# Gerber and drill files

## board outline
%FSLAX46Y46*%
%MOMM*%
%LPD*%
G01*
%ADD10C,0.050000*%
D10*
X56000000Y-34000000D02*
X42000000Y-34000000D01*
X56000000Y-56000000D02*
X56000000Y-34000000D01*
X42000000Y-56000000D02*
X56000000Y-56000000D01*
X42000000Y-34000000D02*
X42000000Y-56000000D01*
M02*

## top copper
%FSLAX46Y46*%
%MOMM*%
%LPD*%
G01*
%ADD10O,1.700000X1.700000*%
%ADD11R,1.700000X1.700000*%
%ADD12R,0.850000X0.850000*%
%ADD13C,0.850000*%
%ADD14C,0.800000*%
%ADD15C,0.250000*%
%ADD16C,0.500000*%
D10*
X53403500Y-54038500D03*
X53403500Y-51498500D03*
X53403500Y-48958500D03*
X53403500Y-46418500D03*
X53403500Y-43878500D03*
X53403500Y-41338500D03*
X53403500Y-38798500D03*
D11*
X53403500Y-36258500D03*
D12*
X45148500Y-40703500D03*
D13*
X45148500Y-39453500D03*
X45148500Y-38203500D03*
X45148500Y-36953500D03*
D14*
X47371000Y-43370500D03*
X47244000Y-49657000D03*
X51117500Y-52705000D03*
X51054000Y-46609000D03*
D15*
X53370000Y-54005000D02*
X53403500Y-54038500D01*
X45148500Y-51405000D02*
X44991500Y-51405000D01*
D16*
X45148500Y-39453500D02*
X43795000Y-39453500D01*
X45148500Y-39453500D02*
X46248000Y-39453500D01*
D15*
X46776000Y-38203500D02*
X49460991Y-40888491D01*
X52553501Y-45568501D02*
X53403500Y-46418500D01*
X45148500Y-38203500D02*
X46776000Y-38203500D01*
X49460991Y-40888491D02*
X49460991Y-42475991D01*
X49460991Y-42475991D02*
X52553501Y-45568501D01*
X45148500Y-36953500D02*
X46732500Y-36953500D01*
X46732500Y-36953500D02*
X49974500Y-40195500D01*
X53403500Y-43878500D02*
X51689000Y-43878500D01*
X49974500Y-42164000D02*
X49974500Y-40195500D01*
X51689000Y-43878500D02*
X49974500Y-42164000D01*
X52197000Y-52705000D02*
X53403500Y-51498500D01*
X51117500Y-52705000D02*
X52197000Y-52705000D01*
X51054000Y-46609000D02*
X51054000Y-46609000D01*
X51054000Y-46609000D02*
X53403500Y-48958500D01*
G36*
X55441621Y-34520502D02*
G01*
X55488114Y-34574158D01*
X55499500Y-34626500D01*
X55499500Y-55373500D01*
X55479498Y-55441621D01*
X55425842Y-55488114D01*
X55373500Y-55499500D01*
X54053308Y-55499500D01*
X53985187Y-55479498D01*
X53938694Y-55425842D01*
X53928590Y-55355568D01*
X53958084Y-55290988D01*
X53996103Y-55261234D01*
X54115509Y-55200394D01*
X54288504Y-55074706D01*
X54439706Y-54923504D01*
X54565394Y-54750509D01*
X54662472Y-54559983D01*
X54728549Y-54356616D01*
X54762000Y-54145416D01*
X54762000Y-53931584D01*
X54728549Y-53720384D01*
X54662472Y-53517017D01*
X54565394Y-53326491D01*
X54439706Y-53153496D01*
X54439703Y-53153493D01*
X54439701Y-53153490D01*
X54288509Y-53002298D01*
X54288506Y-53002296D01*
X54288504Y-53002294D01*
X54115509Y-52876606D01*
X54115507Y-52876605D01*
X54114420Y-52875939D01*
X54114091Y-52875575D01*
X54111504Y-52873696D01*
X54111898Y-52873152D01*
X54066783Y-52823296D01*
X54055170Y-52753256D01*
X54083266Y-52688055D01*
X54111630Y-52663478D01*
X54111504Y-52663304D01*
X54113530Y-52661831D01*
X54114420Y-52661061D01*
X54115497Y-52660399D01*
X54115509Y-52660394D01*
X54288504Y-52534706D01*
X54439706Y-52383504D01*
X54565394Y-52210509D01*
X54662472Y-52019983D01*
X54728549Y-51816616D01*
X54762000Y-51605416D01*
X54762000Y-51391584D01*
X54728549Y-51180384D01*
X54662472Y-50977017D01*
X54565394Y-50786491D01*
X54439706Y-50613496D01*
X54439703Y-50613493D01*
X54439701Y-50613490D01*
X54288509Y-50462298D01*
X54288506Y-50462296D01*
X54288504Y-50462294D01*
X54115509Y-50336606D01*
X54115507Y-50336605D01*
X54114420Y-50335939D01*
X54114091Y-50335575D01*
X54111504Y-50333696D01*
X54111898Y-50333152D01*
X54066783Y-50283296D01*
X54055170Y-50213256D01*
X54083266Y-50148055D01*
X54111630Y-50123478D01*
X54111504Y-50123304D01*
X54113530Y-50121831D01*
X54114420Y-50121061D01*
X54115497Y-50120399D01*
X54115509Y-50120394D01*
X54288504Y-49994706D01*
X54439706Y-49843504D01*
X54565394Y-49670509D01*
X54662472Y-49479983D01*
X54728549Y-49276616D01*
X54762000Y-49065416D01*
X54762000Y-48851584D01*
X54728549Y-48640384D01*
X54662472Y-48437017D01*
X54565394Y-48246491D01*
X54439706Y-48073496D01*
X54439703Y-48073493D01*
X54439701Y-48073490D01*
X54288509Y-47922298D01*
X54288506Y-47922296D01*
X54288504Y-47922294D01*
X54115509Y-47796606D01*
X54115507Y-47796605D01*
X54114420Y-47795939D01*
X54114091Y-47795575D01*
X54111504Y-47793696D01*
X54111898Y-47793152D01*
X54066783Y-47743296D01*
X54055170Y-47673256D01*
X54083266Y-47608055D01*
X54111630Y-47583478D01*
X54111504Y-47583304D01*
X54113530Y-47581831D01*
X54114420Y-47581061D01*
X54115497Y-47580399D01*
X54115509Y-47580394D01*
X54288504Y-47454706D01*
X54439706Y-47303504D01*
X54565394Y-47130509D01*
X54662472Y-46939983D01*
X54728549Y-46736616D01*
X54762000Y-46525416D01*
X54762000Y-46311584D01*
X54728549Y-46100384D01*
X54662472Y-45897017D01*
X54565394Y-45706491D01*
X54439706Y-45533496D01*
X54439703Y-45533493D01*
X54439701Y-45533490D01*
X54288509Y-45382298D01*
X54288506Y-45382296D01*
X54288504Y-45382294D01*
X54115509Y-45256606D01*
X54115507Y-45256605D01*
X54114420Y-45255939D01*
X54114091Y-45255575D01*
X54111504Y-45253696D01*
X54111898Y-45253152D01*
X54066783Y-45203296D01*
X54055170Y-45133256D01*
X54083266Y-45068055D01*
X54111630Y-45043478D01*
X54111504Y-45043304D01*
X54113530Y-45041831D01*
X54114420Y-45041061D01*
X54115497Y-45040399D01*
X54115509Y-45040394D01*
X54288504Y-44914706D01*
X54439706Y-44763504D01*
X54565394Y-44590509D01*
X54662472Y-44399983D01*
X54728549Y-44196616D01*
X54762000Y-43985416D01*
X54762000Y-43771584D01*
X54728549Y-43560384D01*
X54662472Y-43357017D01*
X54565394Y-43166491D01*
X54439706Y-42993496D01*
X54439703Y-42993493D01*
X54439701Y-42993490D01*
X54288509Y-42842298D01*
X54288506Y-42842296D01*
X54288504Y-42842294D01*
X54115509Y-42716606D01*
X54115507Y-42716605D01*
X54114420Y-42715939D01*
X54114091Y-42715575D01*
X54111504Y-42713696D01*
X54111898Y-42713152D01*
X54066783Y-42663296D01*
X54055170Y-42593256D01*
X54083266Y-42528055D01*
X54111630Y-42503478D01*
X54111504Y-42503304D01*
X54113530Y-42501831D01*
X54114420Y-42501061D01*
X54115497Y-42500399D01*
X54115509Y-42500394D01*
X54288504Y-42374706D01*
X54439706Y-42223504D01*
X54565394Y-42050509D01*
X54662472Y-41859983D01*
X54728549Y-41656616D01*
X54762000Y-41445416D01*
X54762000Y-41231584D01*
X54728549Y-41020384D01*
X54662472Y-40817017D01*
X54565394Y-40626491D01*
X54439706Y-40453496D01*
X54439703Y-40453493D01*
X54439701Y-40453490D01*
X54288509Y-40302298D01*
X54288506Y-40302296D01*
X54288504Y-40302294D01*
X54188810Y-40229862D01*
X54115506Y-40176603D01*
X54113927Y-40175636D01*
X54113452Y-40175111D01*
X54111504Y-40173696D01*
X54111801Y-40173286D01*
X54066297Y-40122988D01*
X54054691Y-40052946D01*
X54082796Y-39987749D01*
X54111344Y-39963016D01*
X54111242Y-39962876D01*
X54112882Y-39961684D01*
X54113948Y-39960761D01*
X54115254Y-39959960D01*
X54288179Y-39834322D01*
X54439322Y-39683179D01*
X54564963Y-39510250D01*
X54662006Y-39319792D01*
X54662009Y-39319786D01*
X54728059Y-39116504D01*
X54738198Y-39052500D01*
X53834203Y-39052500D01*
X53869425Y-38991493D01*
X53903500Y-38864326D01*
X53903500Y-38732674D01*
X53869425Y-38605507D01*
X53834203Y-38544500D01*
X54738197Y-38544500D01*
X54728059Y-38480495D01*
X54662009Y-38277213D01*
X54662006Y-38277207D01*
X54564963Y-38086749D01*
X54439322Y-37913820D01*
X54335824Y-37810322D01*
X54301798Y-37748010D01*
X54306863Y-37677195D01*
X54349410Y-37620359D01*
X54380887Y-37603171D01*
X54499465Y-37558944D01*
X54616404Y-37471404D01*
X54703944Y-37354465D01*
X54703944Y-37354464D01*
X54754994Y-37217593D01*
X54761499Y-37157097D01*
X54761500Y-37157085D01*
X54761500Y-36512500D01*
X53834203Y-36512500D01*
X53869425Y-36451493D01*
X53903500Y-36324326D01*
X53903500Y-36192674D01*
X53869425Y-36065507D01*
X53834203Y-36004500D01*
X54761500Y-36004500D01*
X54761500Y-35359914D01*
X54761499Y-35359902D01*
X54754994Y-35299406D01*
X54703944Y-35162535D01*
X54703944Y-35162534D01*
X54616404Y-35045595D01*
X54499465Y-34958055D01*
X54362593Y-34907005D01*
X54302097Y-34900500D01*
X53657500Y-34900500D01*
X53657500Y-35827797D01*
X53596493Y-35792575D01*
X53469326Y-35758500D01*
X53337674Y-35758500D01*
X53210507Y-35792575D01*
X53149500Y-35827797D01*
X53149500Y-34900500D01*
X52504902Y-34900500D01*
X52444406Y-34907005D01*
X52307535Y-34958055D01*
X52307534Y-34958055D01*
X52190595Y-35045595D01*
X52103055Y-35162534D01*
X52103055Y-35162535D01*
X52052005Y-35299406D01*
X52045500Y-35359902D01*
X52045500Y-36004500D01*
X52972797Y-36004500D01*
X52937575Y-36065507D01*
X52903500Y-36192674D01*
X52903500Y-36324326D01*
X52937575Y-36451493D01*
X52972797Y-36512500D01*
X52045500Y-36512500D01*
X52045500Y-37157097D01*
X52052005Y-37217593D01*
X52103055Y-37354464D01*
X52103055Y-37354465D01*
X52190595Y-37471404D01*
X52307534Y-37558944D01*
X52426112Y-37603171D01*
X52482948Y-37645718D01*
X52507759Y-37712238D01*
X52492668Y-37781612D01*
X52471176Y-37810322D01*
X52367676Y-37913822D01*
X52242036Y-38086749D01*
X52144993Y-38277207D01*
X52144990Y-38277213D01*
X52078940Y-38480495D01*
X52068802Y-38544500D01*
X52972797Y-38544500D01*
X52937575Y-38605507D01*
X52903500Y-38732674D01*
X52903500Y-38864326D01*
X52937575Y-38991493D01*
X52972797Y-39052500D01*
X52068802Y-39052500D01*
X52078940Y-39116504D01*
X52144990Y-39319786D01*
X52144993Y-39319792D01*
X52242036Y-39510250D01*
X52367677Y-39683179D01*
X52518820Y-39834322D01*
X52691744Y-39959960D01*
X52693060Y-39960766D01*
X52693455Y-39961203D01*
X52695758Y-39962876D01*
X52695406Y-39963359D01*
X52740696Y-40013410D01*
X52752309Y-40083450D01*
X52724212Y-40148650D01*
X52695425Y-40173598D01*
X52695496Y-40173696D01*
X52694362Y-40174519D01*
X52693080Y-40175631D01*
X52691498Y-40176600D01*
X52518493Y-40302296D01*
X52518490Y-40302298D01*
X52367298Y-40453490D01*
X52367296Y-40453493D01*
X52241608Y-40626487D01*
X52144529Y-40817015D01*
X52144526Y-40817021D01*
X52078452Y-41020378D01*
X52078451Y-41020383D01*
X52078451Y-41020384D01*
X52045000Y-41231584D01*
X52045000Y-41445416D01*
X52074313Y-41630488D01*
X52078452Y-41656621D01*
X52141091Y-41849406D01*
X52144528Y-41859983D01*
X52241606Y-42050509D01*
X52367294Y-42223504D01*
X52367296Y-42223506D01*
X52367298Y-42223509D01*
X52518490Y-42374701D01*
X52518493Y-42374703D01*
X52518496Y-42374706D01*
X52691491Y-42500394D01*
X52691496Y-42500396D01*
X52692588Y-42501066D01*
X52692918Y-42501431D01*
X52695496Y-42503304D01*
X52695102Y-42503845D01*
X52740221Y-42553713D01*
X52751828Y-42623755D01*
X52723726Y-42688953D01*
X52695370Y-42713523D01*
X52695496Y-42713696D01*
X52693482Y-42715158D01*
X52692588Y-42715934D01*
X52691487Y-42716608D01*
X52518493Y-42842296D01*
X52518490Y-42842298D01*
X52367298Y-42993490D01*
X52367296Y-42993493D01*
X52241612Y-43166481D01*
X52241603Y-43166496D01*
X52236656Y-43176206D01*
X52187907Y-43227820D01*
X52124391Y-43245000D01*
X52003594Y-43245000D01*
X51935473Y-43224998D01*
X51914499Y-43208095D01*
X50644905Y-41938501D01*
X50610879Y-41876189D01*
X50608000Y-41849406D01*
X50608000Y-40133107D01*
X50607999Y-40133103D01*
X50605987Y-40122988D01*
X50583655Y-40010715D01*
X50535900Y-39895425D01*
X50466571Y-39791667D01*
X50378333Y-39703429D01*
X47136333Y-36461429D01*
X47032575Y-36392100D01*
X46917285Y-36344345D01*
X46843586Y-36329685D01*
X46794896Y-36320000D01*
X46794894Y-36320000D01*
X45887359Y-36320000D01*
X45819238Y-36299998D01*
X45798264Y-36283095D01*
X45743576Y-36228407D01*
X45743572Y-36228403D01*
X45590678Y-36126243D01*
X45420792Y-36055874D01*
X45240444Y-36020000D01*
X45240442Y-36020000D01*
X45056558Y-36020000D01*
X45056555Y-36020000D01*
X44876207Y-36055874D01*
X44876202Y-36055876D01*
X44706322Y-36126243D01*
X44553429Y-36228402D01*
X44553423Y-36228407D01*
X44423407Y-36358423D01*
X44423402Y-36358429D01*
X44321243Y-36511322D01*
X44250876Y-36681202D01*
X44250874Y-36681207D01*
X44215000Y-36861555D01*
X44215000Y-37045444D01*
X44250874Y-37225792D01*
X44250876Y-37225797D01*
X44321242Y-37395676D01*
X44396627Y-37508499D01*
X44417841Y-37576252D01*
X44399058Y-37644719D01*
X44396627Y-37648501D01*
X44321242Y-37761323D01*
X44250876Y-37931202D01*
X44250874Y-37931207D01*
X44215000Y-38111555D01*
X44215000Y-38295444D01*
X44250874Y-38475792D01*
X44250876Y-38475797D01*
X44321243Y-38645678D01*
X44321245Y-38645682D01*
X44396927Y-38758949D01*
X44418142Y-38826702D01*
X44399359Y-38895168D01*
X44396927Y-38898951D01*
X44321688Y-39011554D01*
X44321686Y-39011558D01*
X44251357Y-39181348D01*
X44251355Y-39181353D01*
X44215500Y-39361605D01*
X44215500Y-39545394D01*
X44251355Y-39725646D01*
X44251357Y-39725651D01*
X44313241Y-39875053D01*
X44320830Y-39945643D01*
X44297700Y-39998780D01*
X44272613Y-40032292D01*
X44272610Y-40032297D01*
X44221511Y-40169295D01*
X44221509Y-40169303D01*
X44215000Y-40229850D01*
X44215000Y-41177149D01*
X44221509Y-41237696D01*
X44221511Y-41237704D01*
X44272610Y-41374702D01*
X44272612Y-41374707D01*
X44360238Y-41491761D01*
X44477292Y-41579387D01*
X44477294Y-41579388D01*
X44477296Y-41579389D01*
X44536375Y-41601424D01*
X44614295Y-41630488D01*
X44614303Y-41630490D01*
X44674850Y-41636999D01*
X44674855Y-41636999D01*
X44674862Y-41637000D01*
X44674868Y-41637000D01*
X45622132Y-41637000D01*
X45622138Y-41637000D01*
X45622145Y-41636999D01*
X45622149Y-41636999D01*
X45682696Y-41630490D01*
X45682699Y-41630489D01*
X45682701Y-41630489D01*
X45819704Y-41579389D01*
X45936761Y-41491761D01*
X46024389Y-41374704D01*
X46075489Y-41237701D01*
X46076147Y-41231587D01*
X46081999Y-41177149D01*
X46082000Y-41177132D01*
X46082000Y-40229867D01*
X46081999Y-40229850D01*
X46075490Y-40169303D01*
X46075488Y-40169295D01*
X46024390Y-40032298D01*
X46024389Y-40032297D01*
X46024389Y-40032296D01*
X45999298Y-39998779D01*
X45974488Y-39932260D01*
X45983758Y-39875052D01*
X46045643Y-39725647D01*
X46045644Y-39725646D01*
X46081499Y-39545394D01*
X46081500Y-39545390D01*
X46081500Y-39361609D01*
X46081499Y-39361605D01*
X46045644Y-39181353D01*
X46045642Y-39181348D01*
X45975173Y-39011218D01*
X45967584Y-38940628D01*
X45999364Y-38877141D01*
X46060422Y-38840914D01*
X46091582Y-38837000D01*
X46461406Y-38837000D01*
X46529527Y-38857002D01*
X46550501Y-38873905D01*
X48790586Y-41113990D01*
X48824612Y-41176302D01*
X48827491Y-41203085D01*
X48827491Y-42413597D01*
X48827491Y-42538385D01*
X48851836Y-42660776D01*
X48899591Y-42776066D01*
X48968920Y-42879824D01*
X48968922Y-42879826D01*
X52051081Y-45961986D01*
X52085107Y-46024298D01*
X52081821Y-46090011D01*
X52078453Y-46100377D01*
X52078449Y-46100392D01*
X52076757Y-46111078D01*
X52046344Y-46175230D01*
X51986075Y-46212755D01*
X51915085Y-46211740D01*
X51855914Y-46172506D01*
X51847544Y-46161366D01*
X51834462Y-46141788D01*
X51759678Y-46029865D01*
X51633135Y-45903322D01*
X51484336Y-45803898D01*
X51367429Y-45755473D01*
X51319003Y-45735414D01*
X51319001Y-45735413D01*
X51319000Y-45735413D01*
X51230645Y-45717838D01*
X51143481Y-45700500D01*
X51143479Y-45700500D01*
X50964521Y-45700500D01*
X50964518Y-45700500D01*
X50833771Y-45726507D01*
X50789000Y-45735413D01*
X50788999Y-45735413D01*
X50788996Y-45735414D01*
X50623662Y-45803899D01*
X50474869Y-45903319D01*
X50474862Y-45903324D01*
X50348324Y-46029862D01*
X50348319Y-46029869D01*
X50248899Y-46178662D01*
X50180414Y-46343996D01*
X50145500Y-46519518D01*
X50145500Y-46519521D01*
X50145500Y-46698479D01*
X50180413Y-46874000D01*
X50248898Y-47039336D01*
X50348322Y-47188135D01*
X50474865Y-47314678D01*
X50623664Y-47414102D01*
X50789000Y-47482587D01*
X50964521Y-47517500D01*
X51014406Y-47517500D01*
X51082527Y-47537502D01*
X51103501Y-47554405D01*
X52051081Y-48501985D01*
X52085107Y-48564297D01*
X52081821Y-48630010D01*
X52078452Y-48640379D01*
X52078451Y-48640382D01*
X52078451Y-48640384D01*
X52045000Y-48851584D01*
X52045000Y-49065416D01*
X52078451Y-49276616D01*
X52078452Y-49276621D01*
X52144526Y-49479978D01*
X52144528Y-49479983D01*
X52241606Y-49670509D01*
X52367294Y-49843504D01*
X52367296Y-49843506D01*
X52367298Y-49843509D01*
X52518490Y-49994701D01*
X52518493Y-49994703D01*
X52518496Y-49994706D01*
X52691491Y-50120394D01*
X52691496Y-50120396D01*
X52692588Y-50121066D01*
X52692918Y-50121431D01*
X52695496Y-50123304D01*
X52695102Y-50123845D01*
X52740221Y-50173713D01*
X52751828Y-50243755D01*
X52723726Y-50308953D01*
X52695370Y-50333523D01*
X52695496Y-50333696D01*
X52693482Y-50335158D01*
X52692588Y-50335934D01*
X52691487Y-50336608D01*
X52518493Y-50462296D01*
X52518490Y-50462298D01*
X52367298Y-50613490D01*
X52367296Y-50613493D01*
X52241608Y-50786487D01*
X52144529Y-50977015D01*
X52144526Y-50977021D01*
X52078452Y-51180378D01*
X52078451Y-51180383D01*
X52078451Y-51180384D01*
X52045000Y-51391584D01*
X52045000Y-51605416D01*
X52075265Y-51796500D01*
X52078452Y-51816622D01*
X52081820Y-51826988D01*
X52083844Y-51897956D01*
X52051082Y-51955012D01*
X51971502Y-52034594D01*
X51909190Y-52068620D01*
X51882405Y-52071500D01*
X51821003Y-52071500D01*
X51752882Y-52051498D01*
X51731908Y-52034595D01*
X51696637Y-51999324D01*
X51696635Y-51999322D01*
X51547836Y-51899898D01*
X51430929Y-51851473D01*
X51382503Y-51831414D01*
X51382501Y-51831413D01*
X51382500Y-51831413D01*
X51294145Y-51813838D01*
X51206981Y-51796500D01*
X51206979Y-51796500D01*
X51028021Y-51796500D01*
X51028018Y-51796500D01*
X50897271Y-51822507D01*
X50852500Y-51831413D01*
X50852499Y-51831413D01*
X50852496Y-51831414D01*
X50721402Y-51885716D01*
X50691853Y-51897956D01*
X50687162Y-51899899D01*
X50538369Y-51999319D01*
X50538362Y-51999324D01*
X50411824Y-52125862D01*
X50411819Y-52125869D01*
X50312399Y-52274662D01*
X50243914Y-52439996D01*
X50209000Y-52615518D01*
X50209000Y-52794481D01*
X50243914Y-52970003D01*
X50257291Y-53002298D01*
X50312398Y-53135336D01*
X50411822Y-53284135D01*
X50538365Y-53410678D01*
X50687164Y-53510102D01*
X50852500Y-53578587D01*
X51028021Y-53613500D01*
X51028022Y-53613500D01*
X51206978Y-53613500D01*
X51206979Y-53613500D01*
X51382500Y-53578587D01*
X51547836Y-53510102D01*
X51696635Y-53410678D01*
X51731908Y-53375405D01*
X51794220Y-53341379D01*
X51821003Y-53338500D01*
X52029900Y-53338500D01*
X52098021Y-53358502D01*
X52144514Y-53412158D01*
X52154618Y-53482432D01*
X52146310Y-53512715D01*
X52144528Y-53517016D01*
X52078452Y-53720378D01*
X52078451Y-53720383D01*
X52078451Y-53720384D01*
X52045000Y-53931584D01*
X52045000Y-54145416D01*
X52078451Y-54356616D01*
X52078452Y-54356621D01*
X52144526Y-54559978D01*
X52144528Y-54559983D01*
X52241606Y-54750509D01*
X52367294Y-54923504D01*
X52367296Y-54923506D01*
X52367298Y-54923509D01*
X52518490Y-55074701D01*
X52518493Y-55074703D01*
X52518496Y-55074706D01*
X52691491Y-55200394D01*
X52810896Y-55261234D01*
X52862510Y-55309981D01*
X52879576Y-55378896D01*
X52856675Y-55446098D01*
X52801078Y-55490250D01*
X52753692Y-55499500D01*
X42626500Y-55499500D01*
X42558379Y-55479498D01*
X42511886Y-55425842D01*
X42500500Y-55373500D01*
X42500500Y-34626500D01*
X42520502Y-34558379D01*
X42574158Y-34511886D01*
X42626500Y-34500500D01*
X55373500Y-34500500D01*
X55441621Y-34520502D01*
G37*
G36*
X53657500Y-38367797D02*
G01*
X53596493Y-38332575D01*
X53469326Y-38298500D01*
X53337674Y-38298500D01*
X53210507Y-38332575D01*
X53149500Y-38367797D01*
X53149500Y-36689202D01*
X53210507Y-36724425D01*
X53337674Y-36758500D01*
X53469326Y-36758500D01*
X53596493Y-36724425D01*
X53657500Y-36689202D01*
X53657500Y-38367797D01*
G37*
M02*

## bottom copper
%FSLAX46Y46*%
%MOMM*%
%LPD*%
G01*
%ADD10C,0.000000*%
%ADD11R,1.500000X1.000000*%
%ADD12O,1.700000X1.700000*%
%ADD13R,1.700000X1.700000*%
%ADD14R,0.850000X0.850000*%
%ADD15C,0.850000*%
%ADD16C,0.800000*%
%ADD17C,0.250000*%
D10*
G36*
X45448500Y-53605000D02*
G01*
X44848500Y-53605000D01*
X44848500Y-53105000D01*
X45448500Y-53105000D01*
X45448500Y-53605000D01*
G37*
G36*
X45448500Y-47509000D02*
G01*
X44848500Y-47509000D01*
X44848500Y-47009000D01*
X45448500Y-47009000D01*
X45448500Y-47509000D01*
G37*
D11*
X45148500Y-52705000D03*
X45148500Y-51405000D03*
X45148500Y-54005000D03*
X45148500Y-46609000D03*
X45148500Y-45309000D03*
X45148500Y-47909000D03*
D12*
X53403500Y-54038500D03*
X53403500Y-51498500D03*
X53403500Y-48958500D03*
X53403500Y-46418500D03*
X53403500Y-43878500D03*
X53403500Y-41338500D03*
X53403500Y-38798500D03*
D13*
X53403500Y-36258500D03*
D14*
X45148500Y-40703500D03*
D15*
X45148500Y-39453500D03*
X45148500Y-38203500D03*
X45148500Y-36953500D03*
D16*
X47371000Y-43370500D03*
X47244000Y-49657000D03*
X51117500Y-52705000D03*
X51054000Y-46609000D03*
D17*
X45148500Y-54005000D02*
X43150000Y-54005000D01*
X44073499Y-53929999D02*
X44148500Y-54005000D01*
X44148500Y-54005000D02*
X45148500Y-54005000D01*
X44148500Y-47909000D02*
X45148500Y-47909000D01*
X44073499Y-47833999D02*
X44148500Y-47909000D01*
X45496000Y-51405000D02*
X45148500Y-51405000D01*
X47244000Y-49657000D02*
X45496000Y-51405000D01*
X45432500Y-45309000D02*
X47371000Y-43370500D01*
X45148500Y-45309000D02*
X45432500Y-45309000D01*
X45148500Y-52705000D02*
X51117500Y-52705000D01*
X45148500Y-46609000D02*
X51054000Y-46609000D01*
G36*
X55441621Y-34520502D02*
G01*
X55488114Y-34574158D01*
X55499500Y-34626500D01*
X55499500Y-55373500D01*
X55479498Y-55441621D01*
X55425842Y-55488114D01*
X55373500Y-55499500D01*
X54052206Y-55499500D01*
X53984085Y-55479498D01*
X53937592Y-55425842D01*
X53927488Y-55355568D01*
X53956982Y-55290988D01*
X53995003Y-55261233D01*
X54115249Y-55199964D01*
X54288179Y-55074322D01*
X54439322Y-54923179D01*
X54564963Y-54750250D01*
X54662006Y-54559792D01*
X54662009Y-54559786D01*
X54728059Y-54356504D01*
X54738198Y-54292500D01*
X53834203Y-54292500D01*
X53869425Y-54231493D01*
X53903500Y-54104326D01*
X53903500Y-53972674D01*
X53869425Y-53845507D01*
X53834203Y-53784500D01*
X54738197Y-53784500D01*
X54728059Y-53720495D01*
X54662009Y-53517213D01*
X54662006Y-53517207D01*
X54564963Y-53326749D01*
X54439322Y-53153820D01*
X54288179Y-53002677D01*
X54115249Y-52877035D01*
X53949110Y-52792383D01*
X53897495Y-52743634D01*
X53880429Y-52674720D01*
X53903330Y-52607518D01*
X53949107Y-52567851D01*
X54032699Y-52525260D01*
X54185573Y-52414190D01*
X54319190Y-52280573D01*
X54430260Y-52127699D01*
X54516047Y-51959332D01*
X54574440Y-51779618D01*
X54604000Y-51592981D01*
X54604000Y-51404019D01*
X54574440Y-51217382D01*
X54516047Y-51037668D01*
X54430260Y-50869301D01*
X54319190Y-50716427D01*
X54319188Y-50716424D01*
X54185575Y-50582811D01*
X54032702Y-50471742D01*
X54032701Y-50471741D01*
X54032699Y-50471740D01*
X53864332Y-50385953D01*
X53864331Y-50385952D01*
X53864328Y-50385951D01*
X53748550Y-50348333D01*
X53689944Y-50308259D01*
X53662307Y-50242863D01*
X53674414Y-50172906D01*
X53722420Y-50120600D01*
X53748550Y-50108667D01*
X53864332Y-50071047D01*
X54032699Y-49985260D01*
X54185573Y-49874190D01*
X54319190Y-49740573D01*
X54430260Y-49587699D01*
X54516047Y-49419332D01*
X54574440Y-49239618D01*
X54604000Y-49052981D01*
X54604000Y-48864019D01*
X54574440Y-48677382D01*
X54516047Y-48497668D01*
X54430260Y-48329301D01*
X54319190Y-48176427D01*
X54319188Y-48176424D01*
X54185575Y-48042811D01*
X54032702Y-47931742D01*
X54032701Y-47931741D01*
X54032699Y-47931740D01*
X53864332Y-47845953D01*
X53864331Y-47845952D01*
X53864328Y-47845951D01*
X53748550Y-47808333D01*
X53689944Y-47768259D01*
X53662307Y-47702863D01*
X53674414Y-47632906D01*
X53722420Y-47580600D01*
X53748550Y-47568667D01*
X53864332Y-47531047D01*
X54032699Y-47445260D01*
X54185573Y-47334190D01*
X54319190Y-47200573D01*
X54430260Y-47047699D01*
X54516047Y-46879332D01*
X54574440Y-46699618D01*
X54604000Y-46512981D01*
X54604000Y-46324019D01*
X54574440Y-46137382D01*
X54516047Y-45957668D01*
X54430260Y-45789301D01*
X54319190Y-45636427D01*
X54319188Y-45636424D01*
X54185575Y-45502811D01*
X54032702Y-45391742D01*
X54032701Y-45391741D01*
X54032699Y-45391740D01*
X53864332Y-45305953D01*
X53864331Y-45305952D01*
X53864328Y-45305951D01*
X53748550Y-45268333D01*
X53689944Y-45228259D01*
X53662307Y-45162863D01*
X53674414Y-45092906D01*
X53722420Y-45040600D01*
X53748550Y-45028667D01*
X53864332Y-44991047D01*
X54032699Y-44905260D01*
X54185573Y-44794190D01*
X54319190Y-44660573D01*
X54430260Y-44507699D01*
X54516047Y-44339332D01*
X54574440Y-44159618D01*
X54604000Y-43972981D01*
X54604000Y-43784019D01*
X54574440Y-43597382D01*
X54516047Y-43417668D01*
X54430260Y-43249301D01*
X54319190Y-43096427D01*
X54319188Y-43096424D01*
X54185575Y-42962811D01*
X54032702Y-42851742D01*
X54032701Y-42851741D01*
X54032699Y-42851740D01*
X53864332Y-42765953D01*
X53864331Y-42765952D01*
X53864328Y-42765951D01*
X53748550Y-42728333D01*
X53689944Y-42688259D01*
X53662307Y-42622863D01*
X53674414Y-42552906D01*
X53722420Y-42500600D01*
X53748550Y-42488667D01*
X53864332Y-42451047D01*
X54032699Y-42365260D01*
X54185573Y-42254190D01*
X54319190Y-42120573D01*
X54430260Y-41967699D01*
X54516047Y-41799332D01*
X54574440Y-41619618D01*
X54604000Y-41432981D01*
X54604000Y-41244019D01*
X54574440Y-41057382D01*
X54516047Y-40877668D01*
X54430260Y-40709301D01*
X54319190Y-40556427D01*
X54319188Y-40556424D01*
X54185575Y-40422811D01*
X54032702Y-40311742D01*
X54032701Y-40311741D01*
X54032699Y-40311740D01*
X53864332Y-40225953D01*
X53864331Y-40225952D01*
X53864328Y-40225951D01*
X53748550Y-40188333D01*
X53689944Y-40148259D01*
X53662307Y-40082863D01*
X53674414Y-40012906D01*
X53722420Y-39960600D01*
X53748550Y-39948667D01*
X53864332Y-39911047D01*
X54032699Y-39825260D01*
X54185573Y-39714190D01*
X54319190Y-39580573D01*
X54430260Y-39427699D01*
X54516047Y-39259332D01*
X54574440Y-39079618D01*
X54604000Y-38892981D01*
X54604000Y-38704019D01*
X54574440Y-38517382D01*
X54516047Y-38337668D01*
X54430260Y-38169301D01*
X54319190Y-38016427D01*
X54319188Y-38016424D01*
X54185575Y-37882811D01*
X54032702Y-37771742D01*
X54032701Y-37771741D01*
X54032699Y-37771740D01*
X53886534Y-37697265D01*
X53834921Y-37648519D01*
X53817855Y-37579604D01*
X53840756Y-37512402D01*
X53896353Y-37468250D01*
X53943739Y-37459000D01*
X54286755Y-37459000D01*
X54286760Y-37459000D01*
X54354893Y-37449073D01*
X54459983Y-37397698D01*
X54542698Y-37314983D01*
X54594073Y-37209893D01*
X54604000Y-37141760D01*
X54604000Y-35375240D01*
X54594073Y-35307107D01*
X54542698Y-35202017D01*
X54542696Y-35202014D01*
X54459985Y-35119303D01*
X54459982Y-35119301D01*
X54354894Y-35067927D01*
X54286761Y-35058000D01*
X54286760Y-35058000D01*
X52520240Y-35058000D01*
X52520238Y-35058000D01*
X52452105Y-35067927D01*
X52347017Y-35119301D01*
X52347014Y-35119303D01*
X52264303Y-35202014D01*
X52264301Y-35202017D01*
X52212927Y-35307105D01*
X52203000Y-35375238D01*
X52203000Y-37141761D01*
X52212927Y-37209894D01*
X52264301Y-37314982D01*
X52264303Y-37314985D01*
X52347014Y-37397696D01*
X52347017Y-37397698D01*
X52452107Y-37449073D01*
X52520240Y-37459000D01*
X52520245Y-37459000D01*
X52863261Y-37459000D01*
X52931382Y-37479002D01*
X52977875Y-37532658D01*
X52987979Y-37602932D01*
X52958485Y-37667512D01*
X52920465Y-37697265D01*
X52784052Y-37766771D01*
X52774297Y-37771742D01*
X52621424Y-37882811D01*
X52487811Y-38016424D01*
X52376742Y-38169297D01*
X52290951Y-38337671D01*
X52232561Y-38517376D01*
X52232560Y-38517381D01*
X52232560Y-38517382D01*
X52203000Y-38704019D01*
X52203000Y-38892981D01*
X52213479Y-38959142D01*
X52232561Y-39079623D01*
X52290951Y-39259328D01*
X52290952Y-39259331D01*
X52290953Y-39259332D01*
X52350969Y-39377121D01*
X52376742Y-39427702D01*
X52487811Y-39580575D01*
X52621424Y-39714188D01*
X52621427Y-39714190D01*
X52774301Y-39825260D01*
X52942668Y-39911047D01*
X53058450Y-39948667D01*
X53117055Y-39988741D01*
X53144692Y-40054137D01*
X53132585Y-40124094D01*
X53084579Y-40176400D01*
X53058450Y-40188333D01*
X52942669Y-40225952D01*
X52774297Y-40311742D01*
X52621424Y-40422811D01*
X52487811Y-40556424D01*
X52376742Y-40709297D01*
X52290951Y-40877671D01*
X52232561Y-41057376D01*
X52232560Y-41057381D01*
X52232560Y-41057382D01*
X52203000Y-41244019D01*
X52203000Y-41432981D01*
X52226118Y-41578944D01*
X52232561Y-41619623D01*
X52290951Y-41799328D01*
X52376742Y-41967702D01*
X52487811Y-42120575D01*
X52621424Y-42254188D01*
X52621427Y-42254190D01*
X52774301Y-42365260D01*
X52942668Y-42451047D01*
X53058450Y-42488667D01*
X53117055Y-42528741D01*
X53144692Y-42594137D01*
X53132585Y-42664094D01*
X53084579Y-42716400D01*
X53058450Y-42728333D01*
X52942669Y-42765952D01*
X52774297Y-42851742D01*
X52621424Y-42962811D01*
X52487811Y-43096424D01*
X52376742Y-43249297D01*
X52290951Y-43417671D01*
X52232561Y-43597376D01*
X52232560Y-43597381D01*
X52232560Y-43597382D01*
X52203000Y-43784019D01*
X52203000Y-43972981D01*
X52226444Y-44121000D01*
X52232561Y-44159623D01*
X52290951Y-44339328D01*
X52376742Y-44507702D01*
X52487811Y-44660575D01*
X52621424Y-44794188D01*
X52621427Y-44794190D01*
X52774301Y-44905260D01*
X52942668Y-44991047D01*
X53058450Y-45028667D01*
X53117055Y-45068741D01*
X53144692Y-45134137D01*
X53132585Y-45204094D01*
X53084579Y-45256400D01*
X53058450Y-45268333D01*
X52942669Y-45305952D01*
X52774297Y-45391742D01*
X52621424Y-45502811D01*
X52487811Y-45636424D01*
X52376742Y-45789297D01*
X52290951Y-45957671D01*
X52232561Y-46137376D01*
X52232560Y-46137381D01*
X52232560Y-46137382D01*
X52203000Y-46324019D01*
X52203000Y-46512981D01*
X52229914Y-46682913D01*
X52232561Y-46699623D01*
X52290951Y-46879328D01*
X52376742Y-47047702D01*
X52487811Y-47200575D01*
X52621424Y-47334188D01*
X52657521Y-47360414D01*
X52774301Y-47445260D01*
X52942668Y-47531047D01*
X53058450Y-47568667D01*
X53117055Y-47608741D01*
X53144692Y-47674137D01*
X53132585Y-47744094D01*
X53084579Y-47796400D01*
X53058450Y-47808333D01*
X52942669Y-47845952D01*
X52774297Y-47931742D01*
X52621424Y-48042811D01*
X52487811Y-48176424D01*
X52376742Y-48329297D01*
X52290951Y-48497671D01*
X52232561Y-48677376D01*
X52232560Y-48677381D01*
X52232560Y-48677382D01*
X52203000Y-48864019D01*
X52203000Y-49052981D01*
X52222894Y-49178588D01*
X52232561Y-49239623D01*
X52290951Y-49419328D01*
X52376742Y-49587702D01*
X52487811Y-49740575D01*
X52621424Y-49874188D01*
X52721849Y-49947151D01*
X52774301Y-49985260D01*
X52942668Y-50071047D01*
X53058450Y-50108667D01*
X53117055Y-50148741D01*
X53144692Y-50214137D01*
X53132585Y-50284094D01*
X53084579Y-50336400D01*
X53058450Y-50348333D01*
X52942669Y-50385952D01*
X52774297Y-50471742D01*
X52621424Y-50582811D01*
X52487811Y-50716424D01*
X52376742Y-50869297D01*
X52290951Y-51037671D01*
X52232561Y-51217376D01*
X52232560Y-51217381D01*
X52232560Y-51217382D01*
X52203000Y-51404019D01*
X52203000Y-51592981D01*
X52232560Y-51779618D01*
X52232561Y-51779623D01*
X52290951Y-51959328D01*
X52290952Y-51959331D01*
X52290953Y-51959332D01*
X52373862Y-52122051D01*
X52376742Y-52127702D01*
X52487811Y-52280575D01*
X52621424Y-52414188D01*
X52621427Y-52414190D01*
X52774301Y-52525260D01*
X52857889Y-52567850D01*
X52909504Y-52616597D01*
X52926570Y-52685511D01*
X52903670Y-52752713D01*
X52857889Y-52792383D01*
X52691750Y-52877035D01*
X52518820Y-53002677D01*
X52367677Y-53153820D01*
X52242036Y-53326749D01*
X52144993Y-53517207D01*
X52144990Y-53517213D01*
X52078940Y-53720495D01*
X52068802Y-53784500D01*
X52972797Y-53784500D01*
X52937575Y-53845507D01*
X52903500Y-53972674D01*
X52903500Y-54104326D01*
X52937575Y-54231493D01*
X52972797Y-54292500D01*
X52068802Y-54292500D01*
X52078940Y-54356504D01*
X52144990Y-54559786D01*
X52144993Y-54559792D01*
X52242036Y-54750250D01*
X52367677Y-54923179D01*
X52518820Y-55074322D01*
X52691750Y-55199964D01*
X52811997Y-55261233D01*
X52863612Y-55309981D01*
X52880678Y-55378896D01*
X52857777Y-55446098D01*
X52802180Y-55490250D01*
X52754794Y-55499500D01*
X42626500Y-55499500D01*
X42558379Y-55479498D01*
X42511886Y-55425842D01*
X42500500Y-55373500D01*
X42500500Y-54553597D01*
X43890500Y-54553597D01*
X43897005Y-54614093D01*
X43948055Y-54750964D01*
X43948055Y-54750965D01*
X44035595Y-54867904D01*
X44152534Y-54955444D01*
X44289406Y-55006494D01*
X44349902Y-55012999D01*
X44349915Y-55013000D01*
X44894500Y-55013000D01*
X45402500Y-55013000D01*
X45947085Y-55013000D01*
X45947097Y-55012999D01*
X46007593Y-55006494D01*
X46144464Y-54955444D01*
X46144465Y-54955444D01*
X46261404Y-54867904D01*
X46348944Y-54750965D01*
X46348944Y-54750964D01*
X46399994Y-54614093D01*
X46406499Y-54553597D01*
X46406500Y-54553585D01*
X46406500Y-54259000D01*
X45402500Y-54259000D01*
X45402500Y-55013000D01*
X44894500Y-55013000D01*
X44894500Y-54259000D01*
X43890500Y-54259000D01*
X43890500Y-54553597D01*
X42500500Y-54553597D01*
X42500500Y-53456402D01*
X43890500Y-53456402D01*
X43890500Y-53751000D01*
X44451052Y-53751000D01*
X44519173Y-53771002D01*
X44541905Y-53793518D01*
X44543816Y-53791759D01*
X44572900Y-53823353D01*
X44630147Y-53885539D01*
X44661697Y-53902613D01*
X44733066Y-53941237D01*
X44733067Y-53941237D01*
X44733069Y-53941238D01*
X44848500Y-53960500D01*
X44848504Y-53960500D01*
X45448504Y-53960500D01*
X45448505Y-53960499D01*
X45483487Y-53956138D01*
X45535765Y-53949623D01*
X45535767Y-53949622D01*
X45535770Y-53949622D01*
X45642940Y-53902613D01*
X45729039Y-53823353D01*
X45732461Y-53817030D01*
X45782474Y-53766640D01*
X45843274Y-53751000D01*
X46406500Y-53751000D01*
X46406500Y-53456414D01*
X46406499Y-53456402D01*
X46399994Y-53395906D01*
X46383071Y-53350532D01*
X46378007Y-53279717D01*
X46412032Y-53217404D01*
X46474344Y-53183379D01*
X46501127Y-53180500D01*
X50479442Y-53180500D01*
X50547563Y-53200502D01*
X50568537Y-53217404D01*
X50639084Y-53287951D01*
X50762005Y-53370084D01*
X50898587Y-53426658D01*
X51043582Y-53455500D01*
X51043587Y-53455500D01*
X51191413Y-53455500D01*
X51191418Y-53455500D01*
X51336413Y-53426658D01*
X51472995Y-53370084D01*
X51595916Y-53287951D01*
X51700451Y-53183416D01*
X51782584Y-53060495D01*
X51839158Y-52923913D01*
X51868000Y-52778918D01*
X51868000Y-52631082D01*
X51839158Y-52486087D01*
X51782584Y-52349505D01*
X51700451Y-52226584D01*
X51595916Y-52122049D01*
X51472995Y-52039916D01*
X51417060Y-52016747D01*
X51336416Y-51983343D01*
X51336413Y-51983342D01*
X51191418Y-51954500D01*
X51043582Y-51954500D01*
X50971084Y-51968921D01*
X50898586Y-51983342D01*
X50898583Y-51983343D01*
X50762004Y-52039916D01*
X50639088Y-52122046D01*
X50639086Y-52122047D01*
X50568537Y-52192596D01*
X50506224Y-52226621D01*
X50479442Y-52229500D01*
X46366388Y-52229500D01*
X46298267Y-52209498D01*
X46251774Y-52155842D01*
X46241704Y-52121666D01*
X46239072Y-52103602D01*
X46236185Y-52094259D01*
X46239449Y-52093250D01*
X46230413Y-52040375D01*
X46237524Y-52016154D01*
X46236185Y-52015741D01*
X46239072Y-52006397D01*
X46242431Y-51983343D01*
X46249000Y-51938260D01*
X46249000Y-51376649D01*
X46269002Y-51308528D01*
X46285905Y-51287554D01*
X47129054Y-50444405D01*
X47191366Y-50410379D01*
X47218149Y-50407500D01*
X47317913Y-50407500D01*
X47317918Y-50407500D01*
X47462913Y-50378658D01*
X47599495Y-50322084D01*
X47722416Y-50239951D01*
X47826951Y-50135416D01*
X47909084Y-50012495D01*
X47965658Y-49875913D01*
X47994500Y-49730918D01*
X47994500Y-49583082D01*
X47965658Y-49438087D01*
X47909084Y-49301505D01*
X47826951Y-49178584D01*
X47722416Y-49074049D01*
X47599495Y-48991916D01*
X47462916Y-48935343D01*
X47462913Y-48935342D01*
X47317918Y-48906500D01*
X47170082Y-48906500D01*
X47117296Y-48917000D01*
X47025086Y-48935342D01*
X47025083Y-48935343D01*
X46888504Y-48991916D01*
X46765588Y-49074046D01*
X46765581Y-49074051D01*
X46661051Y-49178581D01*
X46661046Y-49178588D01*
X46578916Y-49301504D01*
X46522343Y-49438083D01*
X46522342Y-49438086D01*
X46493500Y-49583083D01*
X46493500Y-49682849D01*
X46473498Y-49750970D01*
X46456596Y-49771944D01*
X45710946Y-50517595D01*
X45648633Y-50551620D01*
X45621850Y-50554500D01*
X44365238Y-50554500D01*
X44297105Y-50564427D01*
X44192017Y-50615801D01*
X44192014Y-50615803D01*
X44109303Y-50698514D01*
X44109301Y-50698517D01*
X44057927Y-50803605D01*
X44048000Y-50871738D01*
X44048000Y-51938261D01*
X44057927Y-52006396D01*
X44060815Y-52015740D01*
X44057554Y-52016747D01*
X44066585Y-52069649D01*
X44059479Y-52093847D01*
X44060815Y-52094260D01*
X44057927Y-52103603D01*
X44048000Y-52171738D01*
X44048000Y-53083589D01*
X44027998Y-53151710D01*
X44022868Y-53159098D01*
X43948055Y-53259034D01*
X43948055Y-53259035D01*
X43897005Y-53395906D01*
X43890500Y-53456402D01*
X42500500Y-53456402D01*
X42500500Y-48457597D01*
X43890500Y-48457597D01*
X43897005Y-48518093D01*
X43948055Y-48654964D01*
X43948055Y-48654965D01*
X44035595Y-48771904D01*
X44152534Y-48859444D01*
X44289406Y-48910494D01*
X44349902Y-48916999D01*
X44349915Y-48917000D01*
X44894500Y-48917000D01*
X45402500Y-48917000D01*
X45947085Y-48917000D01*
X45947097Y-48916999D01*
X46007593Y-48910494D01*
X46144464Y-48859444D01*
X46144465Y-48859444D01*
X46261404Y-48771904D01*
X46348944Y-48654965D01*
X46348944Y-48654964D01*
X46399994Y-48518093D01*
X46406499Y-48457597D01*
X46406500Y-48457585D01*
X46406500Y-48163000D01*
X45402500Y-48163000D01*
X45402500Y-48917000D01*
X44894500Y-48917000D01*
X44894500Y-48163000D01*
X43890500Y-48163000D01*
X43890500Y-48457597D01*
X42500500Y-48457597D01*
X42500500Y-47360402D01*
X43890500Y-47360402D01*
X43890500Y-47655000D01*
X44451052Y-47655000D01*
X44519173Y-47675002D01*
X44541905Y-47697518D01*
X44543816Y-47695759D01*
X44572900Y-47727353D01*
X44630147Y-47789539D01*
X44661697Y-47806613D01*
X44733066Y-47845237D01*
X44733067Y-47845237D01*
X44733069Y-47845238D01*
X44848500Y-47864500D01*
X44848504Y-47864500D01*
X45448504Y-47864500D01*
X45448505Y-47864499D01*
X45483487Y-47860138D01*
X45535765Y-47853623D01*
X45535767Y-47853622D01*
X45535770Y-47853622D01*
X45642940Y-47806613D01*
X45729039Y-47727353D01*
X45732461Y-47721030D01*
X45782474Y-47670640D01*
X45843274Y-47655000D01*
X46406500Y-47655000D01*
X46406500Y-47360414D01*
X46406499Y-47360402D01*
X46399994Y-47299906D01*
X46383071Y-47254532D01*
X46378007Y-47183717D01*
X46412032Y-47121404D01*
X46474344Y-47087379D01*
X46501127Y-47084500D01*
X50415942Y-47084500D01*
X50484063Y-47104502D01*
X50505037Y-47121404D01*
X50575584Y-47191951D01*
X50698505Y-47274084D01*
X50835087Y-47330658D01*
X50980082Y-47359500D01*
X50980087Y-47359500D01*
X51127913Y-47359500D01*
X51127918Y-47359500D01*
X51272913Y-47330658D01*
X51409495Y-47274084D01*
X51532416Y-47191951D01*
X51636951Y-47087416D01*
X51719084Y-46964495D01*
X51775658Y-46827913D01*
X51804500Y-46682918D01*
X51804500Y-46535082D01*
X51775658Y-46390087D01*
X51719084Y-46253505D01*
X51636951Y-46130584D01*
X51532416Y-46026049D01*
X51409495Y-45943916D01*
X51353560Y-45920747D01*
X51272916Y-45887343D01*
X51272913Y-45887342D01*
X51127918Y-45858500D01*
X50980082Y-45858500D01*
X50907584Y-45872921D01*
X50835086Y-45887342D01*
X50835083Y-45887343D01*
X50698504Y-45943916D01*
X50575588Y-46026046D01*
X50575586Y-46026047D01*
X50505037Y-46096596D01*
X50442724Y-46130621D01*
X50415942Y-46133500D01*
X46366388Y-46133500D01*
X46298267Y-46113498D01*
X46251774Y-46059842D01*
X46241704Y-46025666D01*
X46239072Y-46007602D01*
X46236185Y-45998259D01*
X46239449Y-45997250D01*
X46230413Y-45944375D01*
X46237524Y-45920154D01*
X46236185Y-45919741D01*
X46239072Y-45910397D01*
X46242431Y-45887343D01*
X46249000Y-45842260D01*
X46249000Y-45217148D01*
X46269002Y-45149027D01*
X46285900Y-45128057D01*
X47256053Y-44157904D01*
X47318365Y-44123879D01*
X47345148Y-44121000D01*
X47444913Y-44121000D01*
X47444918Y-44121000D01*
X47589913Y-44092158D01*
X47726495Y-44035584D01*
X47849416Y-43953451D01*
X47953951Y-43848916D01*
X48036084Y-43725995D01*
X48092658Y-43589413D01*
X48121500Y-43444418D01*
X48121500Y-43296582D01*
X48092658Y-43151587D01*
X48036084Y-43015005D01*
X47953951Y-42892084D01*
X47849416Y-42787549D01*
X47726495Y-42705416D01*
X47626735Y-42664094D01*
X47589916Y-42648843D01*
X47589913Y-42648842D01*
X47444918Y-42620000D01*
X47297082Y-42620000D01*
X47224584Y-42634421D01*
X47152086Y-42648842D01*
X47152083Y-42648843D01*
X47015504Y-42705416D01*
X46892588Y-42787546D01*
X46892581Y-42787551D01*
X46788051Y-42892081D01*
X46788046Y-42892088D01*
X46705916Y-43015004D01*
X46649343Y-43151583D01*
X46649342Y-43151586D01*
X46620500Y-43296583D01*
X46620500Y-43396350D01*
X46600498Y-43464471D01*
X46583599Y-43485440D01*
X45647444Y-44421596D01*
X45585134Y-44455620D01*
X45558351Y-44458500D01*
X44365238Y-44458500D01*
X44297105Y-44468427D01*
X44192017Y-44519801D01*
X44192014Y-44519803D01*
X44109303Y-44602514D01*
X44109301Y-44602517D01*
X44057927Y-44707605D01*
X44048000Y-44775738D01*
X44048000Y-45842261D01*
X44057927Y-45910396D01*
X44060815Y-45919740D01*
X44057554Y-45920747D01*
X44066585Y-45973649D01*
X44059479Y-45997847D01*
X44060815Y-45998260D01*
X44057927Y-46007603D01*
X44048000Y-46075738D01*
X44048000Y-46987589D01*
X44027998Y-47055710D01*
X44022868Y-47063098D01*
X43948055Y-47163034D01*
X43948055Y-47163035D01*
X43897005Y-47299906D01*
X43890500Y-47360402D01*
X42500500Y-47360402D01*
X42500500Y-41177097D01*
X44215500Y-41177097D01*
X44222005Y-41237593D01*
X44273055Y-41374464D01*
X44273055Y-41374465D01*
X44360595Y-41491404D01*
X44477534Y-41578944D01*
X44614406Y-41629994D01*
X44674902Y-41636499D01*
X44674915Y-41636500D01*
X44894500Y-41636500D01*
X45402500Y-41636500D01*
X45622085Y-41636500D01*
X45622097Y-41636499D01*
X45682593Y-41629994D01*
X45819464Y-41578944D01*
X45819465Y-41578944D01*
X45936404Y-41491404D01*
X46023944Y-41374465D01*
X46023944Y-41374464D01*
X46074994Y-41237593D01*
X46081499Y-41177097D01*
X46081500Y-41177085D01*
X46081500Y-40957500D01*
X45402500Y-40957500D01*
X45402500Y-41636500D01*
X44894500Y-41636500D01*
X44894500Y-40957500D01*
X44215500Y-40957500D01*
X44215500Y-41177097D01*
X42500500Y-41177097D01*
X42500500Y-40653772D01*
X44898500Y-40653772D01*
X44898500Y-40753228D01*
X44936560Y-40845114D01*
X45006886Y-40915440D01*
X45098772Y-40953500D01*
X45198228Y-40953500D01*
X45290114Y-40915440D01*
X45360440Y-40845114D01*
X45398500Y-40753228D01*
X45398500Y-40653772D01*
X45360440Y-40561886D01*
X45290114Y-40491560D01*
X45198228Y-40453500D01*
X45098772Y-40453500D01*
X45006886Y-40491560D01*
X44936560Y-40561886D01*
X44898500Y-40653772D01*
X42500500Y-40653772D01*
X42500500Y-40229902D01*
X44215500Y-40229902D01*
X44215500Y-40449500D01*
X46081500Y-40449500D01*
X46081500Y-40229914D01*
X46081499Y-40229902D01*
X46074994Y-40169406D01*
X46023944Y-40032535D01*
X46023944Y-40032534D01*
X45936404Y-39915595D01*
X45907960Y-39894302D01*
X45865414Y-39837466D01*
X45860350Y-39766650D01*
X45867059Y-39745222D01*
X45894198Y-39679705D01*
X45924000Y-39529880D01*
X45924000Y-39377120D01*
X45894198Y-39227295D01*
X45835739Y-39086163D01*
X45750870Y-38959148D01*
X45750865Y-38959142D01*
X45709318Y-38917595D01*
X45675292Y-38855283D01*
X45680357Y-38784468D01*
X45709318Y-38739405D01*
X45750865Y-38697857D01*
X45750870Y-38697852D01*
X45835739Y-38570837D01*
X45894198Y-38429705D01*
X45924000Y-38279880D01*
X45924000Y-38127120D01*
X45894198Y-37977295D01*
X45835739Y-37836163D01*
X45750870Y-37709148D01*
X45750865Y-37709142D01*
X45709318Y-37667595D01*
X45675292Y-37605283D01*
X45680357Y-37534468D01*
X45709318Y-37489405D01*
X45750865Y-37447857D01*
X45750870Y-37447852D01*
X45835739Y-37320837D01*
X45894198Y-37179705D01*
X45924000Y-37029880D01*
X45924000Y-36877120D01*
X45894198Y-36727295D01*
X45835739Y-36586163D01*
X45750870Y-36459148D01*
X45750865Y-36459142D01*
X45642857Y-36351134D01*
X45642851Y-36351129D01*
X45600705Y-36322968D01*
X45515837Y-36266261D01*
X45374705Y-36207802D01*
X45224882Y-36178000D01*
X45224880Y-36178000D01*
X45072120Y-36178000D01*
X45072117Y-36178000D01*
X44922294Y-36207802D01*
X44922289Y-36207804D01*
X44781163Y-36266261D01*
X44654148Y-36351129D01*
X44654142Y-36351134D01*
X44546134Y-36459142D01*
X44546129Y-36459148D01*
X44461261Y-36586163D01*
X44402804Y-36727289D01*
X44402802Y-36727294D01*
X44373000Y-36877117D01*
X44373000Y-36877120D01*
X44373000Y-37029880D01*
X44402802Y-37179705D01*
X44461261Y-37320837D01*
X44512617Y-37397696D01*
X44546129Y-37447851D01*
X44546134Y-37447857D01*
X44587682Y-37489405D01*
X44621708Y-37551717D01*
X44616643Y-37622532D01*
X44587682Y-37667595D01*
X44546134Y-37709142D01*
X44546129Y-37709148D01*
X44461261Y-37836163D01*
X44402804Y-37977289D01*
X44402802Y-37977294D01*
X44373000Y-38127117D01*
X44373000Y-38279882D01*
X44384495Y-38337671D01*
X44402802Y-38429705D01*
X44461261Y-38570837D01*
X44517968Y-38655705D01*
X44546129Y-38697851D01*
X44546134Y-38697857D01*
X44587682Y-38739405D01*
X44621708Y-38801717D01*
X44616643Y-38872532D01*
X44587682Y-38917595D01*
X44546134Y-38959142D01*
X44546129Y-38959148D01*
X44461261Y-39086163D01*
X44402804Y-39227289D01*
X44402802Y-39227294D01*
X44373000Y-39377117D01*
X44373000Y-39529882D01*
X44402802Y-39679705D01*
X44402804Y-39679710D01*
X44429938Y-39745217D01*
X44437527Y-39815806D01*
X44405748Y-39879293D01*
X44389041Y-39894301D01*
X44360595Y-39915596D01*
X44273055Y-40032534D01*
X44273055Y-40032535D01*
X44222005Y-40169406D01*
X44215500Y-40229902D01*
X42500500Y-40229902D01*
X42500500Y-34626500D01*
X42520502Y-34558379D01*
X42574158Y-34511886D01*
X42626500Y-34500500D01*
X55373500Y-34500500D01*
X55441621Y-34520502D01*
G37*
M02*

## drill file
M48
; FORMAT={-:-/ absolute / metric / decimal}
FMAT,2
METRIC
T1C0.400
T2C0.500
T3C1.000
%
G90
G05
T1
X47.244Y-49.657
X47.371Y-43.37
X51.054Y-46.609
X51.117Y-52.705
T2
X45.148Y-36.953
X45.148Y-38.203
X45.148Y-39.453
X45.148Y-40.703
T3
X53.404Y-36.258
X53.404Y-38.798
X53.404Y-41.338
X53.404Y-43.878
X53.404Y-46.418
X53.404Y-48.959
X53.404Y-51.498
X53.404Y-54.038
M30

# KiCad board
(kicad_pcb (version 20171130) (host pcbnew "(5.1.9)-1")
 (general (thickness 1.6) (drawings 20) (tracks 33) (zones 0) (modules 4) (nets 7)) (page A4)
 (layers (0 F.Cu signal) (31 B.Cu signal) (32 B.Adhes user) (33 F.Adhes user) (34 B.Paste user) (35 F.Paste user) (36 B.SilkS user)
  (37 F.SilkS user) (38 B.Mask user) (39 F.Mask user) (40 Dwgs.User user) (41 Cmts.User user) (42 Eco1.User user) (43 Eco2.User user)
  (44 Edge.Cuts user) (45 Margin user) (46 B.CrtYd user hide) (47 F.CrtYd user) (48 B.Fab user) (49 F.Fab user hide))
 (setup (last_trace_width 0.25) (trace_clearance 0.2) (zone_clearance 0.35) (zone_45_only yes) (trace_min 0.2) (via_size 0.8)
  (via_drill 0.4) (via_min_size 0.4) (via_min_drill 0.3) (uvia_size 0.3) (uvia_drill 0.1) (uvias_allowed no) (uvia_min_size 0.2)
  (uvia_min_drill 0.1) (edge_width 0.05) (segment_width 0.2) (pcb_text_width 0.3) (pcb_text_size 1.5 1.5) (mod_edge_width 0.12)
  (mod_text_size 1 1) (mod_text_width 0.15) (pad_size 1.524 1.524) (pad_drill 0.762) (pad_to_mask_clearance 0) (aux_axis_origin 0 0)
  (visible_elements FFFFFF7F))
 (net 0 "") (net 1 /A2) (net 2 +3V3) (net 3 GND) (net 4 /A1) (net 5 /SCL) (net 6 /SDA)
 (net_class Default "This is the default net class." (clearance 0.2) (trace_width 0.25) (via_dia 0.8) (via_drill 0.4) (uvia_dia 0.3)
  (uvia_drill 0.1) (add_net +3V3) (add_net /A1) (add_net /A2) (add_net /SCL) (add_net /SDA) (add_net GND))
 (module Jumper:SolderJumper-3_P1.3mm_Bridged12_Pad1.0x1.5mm (layer B.Cu) (at 45.1485 52.705 90)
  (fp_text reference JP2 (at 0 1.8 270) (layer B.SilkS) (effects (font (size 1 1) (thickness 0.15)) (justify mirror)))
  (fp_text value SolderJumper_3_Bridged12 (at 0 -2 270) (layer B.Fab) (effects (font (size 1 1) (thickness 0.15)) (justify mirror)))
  (fp_poly (pts (xy -0.9 0.3) (xy -0.4 0.3) (xy -0.4 -0.3) (xy -0.9 -0.3)) (layer B.Cu) (width 0))
  (pad 2 smd rect (at 0 0 90) (size 1 1.5) (layers B.Cu B.Mask) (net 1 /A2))
  (pad 3 smd rect (at 1.3 0 90) (size 1 1.5) (layers B.Cu B.Mask) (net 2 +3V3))
  (pad 1 smd rect (at -1.3 0 90) (size 1 1.5) (layers B.Cu B.Mask) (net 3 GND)))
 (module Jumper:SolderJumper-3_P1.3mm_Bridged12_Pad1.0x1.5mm (layer B.Cu) (at 45.1485 46.609 90)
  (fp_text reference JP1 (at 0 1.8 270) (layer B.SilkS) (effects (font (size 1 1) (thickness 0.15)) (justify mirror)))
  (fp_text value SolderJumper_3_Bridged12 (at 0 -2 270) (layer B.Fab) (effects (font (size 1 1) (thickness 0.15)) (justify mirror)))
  (fp_poly (pts (xy -0.9 0.3) (xy -0.4 0.3) (xy -0.4 -0.3) (xy -0.9 -0.3)) (layer B.Cu) (width 0))
  (pad 2 smd rect (at 0 0 90) (size 1 1.5) (layers B.Cu B.Mask) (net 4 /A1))
  (pad 3 smd rect (at 1.3 0 90) (size 1 1.5) (layers B.Cu B.Mask) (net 2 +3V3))
  (pad 1 smd rect (at -1.3 0 90) (size 1 1.5) (layers B.Cu B.Mask) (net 3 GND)))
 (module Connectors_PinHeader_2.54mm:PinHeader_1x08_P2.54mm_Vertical (layer F.Cu) (at 53.4035 36.2585)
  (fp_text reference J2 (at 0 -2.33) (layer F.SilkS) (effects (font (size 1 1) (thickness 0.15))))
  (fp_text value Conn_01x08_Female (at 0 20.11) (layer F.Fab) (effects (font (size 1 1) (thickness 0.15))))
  (pad 8 thru_hole oval (at 0 17.78) (size 1.7 1.7) (drill 1) (layers *.Cu *.Mask) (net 3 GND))
  (pad 7 thru_hole oval (at 0 15.24) (size 1.7 1.7) (drill 1) (layers *.Cu *.Mask) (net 1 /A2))
  (pad 6 thru_hole oval (at 0 12.7) (size 1.7 1.7) (drill 1) (layers *.Cu *.Mask) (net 4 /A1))
  (pad 5 thru_hole oval (at 0 10.16) (size 1.7 1.7) (drill 1) (layers *.Cu *.Mask) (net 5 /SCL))
  (pad 4 thru_hole oval (at 0 7.62) (size 1.7 1.7) (drill 1) (layers *.Cu *.Mask) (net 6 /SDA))
  (pad 3 thru_hole oval (at 0 5.08) (size 1.7 1.7) (drill 1) (layers *.Cu *.Mask))
  (pad 2 thru_hole oval (at 0 2.54) (size 1.7 1.7) (drill 1) (layers *.Cu *.Mask) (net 2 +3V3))
  (pad 1 thru_hole rect (at 0 0) (size 1.7 1.7) (drill 1) (layers *.Cu *.Mask) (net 2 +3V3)))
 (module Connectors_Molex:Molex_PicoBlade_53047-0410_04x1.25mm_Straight (layer B.Cu) (at 45.1485 40.7035 90)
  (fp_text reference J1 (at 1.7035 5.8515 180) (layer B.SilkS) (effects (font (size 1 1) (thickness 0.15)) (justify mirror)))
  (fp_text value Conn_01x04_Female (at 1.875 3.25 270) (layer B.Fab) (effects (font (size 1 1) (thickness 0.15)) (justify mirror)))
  (pad 1 thru_hole rect (at 0 0 90) (size 0.85 0.85) (drill 0.5) (layers *.Cu *.Mask) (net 3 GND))
  (pad 2 thru_hole circle (at 1.25 0 90) (size 0.85 0.85) (drill 0.5) (layers *.Cu *.Mask) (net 2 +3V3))
  (pad 3 thru_hole circle (at 2.5 0 90) (size 0.85 0.85) (drill 0.5) (layers *.Cu *.Mask) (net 5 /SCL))
  (pad 4 thru_hole circle (at 3.75 0 90) (size 0.85 0.85) (drill 0.5) (layers *.Cu *.Mask) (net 6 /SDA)))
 (gr_line (start 56 34) (end 42 34) (layer Edge.Cuts) (width 0.05))
 (gr_line (start 56 56) (end 56 34) (layer Edge.Cuts) (width 0.05))
 (gr_line (start 42 56) (end 56 56) (layer Edge.Cuts) (width 0.05))
 (gr_line (start 42 34) (end 42 56) (layer Edge.Cuts) (width 0.05))
 (segment (start 53.37 54.005) (end 53.4035 54.0385) (width 0.25) (layer F.Cu) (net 3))
 (segment (start 45.1485 54.005) (end 43.15 54.005) (width 0.25) (layer B.Cu) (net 3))
 (segment (start 44.073499 53.929999) (end 44.1485 54.005) (width 0.25) (layer B.Cu) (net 3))
 (segment (start 44.1485 54.005) (end 45.1485 54.005) (width 0.25) (layer B.Cu) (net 3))
 (segment (start 44.1485 47.909) (end 45.1485 47.909) (width 0.25) (layer B.Cu) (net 3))
 (segment (start 44.073499 47.833999) (end 44.1485 47.909) (width 0.25) (layer B.Cu) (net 3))
 (segment (start 45.1485 51.405) (end 44.9915 51.405) (width 0.25) (layer F.Cu) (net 2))
 (segment (start 45.1485 39.4535) (end 43.795 39.4535) (width 0.5) (layer F.Cu) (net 2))
 (segment (start 45.1485 39.4535) (end 46.248 39.4535) (width 0.5) (layer F.Cu) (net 2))
 (via (at 47.371 43.3705) (size 0.8) (drill 0.4) (layers F.Cu B.Cu) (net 2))
 (via (at 47.244 49.657) (size 0.8) (drill 0.4) (layers F.Cu B.Cu) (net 2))
 (segment (start 45.496 51.405) (end 45.1485 51.405) (width 0.25) (layer B.Cu) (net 2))
 (segment (start 47.244 49.657) (end 45.496 51.405) (width 0.25) (layer B.Cu) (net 2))
 (segment (start 45.4325 45.309) (end 47.371 43.3705) (width 0.25) (layer B.Cu) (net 2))
 (segment (start 45.1485 45.309) (end 45.4325 45.309) (width 0.25) (layer B.Cu) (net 2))
 (segment (start 46.776 38.2035) (end 49.460991 40.888491) (width 0.25) (layer F.Cu) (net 5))
 (segment (start 52.553501 45.568501) (end 53.4035 46.4185) (width 0.25) (layer F.Cu) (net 5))
 (segment (start 45.1485 38.2035) (end 46.776 38.2035) (width 0.25) (layer F.Cu) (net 5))
 (segment (start 49.460991 40.888491) (end 49.460991 42.475991) (width 0.25) (layer F.Cu) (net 5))
 (segment (start 49.460991 42.475991) (end 52.553501 45.568501) (width 0.25) (layer F.Cu) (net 5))
 (segment (start 45.1485 36.9535) (end 46.7325 36.9535) (width 0.25) (layer F.Cu) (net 6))
 (segment (start 46.7325 36.9535) (end 49.9745 40.1955) (width 0.25) (layer F.Cu) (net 6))
 (segment (start 53.4035 43.8785) (end 51.689 43.8785) (width 0.25) (layer F.Cu) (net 6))
 (segment (start 49.9745 42.164) (end 49.9745 40.1955) (width 0.25) (layer F.Cu) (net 6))
 (segment (start 51.689 43.8785) (end 49.9745 42.164) (width 0.25) (layer F.Cu) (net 6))
 (segment (start 52.197 52.705) (end 53.4035 51.4985) (width 0.25) (layer F.Cu) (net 1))
 (segment (start 51.1175 52.705) (end 52.197 52.705) (width 0.25) (layer F.Cu) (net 1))
 (via (at 51.1175 52.705) (size 0.8) (drill 0.4) (layers F.Cu B.Cu) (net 1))
 (segment (start 45.1485 52.705) (end 51.1175 52.705) (width 0.25) (layer B.Cu) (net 1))
 (segment (start 51.054 46.609) (end 51.054 46.609) (width 0.25) (layer F.Cu) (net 4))
 (segment (start 51.054 46.609) (end 53.4035 48.9585) (width 0.25) (layer F.Cu) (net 4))
 (via (at 51.054 46.609) (size 0.8) (drill 0.4) (layers F.Cu B.Cu) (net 4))
 (segment (start 45.1485 46.609) (end 51.054 46.609) (width 0.25) (layer B.Cu) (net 4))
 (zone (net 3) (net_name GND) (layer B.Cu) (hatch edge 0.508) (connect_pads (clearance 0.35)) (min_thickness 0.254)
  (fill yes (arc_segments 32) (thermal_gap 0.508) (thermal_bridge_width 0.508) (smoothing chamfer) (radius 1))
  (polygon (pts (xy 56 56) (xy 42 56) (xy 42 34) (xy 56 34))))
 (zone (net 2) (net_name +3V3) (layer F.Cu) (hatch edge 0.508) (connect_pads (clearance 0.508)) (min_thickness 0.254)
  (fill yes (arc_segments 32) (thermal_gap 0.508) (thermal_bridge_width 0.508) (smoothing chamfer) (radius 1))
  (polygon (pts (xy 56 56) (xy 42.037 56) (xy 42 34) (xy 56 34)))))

